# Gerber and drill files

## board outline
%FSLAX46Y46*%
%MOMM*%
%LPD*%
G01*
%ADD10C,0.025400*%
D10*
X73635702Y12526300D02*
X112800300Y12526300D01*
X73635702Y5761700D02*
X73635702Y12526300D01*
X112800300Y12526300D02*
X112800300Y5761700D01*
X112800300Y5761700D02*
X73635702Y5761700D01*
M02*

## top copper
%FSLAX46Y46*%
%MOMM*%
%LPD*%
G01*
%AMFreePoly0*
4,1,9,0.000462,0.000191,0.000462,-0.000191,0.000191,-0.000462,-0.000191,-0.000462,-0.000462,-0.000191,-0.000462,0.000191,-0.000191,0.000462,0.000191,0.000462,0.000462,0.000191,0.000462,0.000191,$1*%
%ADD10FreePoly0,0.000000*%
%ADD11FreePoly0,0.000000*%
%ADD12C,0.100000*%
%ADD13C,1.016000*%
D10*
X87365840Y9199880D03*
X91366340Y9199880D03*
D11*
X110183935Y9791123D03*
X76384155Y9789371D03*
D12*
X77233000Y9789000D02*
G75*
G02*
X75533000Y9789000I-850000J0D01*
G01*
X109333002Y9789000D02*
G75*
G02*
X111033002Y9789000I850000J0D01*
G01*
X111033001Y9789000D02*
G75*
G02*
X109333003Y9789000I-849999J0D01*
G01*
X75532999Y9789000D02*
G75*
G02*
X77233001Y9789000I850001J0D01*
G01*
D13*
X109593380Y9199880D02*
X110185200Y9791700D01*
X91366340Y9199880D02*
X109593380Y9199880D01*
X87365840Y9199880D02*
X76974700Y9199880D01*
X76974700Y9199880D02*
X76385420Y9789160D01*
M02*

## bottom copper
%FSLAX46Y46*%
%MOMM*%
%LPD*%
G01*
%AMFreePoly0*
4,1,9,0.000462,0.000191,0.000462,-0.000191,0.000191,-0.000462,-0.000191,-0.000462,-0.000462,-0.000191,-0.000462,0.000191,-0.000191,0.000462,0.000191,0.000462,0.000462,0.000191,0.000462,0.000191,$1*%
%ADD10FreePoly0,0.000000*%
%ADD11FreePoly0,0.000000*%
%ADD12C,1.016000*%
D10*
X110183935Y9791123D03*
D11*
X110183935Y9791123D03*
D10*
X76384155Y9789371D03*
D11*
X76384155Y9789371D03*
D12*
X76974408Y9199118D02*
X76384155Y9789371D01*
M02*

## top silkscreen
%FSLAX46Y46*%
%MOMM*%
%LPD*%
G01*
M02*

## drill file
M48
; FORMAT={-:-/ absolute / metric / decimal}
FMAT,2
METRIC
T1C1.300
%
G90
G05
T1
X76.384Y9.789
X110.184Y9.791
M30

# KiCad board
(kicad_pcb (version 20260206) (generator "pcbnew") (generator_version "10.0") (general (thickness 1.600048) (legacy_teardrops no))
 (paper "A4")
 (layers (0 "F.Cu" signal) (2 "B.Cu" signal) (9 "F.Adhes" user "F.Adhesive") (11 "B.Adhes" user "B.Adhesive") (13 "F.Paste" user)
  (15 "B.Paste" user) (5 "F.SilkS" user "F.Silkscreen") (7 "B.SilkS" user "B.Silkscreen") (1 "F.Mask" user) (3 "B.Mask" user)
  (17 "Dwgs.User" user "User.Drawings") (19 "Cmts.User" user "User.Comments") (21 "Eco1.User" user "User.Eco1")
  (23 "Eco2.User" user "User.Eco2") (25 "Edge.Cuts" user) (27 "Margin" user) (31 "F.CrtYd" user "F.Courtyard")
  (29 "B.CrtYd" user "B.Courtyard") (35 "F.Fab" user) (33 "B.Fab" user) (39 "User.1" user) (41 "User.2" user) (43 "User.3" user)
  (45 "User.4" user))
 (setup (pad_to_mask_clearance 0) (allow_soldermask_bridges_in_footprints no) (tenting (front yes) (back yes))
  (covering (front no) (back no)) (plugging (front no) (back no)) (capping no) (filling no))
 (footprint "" (layer "F.Cu") (at 0 0)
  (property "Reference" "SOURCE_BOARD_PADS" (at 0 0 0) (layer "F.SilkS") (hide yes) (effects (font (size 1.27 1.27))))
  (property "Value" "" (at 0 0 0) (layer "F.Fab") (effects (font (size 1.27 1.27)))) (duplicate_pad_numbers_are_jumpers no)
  (pad "1" smd custom (at 87.36584 -9.19988) (size 0.001 0.001) (layers "F.Cu" "F.Mask" "F.Paste") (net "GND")
   (options (clearance outline) (anchor circle)) (primitives))
  (pad "2" smd custom (at 91.36634 -9.19988) (size 0.001 0.001) (layers "F.Cu" "F.Mask" "F.Paste") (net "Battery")
   (options (clearance outline) (anchor circle)) (primitives)))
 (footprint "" (layer "B.Cu") (at 110.183935 -9.791123)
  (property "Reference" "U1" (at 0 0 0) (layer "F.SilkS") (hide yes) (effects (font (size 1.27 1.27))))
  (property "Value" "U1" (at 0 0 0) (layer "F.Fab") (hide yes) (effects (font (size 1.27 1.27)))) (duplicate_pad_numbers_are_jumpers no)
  (pad "1" thru_hole custom (at 0 0) (size 0.001 0.001) (drill 1.300023) (layers "*.Cu") (remove_unused_layers no) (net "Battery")
   (options (clearance outline) (anchor circle)) (primitives))
  (pad "1" smd custom (at 0 0) (size 0.001 0.001) (layers "B.Cu" "B.Mask" "B.Paste") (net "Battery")
   (options (clearance outline) (anchor circle)) (primitives)))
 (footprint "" (layer "B.Cu") (at 76.384155 -9.789371)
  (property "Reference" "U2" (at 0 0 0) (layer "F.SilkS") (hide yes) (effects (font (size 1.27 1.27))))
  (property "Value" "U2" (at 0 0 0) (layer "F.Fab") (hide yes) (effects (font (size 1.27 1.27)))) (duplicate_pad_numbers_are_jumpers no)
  (pad "1" thru_hole custom (at 0 0) (size 0.001 0.001) (drill 1.300023) (layers "*.Cu") (remove_unused_layers no) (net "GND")
   (options (clearance outline) (anchor circle)) (primitives))
  (pad "1" smd custom (at 0 0) (size 0.001 0.001) (layers "B.Cu" "B.Mask" "B.Paste") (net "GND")
   (options (clearance outline) (anchor circle)) (primitives)))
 (gr_line (start 73.635702 -12.5263) (end 112.8003 -12.5263) (stroke (width 0.0254) (type default)) (layer "Edge.Cuts"))
 (gr_line (start 73.635702 -5.7617) (end 73.635702 -12.5263) (stroke (width 0.0254) (type default)) (layer "Edge.Cuts"))
 (gr_line (start 112.8003 -12.5263) (end 112.8003 -5.7617) (stroke (width 0.0254) (type default)) (layer "Edge.Cuts"))
 (gr_line (start 112.8003 -5.7617) (end 73.635702 -5.7617) (stroke (width 0.0254) (type default)) (layer "Edge.Cuts"))
 (arc (start 77.233 -9.789) (mid 76.364711 -8.939196) (end 75.532999 -9.789) (width 0.1) (layer "F.Cu") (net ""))
 (arc (start 109.333002 -9.789) (mid 110.20129 -10.638803) (end 111.033001 -9.789) (width 0.1) (layer "F.Cu") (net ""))
 (arc (start 111.033001 -9.789) (mid 110.164713 -8.939197) (end 109.333002 -9.789) (width 0.1) (layer "F.Cu") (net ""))
 (arc (start 75.532999 -9.789) (mid 76.401288 -10.638804) (end 77.233 -9.789) (width 0.1) (layer "F.Cu") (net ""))
 (segment (start 109.59338 -9.19988) (end 110.1852 -9.7917) (width 1.016) (layer "F.Cu") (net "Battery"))
 (segment (start 91.36634 -9.19988) (end 109.59338 -9.19988) (width 1.016) (layer "F.Cu") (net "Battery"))
 (segment (start 87.36584 -9.19988) (end 76.9747 -9.19988) (width 1.016) (layer "F.Cu") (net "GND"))
 (segment (start 76.9747 -9.19988) (end 76.38542 -9.78916) (width 1.016) (layer "F.Cu") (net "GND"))
 (segment (start 76.974408 -9.199118) (end 76.384155 -9.789371) (width 1.016) (layer "B.Cu") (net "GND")))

